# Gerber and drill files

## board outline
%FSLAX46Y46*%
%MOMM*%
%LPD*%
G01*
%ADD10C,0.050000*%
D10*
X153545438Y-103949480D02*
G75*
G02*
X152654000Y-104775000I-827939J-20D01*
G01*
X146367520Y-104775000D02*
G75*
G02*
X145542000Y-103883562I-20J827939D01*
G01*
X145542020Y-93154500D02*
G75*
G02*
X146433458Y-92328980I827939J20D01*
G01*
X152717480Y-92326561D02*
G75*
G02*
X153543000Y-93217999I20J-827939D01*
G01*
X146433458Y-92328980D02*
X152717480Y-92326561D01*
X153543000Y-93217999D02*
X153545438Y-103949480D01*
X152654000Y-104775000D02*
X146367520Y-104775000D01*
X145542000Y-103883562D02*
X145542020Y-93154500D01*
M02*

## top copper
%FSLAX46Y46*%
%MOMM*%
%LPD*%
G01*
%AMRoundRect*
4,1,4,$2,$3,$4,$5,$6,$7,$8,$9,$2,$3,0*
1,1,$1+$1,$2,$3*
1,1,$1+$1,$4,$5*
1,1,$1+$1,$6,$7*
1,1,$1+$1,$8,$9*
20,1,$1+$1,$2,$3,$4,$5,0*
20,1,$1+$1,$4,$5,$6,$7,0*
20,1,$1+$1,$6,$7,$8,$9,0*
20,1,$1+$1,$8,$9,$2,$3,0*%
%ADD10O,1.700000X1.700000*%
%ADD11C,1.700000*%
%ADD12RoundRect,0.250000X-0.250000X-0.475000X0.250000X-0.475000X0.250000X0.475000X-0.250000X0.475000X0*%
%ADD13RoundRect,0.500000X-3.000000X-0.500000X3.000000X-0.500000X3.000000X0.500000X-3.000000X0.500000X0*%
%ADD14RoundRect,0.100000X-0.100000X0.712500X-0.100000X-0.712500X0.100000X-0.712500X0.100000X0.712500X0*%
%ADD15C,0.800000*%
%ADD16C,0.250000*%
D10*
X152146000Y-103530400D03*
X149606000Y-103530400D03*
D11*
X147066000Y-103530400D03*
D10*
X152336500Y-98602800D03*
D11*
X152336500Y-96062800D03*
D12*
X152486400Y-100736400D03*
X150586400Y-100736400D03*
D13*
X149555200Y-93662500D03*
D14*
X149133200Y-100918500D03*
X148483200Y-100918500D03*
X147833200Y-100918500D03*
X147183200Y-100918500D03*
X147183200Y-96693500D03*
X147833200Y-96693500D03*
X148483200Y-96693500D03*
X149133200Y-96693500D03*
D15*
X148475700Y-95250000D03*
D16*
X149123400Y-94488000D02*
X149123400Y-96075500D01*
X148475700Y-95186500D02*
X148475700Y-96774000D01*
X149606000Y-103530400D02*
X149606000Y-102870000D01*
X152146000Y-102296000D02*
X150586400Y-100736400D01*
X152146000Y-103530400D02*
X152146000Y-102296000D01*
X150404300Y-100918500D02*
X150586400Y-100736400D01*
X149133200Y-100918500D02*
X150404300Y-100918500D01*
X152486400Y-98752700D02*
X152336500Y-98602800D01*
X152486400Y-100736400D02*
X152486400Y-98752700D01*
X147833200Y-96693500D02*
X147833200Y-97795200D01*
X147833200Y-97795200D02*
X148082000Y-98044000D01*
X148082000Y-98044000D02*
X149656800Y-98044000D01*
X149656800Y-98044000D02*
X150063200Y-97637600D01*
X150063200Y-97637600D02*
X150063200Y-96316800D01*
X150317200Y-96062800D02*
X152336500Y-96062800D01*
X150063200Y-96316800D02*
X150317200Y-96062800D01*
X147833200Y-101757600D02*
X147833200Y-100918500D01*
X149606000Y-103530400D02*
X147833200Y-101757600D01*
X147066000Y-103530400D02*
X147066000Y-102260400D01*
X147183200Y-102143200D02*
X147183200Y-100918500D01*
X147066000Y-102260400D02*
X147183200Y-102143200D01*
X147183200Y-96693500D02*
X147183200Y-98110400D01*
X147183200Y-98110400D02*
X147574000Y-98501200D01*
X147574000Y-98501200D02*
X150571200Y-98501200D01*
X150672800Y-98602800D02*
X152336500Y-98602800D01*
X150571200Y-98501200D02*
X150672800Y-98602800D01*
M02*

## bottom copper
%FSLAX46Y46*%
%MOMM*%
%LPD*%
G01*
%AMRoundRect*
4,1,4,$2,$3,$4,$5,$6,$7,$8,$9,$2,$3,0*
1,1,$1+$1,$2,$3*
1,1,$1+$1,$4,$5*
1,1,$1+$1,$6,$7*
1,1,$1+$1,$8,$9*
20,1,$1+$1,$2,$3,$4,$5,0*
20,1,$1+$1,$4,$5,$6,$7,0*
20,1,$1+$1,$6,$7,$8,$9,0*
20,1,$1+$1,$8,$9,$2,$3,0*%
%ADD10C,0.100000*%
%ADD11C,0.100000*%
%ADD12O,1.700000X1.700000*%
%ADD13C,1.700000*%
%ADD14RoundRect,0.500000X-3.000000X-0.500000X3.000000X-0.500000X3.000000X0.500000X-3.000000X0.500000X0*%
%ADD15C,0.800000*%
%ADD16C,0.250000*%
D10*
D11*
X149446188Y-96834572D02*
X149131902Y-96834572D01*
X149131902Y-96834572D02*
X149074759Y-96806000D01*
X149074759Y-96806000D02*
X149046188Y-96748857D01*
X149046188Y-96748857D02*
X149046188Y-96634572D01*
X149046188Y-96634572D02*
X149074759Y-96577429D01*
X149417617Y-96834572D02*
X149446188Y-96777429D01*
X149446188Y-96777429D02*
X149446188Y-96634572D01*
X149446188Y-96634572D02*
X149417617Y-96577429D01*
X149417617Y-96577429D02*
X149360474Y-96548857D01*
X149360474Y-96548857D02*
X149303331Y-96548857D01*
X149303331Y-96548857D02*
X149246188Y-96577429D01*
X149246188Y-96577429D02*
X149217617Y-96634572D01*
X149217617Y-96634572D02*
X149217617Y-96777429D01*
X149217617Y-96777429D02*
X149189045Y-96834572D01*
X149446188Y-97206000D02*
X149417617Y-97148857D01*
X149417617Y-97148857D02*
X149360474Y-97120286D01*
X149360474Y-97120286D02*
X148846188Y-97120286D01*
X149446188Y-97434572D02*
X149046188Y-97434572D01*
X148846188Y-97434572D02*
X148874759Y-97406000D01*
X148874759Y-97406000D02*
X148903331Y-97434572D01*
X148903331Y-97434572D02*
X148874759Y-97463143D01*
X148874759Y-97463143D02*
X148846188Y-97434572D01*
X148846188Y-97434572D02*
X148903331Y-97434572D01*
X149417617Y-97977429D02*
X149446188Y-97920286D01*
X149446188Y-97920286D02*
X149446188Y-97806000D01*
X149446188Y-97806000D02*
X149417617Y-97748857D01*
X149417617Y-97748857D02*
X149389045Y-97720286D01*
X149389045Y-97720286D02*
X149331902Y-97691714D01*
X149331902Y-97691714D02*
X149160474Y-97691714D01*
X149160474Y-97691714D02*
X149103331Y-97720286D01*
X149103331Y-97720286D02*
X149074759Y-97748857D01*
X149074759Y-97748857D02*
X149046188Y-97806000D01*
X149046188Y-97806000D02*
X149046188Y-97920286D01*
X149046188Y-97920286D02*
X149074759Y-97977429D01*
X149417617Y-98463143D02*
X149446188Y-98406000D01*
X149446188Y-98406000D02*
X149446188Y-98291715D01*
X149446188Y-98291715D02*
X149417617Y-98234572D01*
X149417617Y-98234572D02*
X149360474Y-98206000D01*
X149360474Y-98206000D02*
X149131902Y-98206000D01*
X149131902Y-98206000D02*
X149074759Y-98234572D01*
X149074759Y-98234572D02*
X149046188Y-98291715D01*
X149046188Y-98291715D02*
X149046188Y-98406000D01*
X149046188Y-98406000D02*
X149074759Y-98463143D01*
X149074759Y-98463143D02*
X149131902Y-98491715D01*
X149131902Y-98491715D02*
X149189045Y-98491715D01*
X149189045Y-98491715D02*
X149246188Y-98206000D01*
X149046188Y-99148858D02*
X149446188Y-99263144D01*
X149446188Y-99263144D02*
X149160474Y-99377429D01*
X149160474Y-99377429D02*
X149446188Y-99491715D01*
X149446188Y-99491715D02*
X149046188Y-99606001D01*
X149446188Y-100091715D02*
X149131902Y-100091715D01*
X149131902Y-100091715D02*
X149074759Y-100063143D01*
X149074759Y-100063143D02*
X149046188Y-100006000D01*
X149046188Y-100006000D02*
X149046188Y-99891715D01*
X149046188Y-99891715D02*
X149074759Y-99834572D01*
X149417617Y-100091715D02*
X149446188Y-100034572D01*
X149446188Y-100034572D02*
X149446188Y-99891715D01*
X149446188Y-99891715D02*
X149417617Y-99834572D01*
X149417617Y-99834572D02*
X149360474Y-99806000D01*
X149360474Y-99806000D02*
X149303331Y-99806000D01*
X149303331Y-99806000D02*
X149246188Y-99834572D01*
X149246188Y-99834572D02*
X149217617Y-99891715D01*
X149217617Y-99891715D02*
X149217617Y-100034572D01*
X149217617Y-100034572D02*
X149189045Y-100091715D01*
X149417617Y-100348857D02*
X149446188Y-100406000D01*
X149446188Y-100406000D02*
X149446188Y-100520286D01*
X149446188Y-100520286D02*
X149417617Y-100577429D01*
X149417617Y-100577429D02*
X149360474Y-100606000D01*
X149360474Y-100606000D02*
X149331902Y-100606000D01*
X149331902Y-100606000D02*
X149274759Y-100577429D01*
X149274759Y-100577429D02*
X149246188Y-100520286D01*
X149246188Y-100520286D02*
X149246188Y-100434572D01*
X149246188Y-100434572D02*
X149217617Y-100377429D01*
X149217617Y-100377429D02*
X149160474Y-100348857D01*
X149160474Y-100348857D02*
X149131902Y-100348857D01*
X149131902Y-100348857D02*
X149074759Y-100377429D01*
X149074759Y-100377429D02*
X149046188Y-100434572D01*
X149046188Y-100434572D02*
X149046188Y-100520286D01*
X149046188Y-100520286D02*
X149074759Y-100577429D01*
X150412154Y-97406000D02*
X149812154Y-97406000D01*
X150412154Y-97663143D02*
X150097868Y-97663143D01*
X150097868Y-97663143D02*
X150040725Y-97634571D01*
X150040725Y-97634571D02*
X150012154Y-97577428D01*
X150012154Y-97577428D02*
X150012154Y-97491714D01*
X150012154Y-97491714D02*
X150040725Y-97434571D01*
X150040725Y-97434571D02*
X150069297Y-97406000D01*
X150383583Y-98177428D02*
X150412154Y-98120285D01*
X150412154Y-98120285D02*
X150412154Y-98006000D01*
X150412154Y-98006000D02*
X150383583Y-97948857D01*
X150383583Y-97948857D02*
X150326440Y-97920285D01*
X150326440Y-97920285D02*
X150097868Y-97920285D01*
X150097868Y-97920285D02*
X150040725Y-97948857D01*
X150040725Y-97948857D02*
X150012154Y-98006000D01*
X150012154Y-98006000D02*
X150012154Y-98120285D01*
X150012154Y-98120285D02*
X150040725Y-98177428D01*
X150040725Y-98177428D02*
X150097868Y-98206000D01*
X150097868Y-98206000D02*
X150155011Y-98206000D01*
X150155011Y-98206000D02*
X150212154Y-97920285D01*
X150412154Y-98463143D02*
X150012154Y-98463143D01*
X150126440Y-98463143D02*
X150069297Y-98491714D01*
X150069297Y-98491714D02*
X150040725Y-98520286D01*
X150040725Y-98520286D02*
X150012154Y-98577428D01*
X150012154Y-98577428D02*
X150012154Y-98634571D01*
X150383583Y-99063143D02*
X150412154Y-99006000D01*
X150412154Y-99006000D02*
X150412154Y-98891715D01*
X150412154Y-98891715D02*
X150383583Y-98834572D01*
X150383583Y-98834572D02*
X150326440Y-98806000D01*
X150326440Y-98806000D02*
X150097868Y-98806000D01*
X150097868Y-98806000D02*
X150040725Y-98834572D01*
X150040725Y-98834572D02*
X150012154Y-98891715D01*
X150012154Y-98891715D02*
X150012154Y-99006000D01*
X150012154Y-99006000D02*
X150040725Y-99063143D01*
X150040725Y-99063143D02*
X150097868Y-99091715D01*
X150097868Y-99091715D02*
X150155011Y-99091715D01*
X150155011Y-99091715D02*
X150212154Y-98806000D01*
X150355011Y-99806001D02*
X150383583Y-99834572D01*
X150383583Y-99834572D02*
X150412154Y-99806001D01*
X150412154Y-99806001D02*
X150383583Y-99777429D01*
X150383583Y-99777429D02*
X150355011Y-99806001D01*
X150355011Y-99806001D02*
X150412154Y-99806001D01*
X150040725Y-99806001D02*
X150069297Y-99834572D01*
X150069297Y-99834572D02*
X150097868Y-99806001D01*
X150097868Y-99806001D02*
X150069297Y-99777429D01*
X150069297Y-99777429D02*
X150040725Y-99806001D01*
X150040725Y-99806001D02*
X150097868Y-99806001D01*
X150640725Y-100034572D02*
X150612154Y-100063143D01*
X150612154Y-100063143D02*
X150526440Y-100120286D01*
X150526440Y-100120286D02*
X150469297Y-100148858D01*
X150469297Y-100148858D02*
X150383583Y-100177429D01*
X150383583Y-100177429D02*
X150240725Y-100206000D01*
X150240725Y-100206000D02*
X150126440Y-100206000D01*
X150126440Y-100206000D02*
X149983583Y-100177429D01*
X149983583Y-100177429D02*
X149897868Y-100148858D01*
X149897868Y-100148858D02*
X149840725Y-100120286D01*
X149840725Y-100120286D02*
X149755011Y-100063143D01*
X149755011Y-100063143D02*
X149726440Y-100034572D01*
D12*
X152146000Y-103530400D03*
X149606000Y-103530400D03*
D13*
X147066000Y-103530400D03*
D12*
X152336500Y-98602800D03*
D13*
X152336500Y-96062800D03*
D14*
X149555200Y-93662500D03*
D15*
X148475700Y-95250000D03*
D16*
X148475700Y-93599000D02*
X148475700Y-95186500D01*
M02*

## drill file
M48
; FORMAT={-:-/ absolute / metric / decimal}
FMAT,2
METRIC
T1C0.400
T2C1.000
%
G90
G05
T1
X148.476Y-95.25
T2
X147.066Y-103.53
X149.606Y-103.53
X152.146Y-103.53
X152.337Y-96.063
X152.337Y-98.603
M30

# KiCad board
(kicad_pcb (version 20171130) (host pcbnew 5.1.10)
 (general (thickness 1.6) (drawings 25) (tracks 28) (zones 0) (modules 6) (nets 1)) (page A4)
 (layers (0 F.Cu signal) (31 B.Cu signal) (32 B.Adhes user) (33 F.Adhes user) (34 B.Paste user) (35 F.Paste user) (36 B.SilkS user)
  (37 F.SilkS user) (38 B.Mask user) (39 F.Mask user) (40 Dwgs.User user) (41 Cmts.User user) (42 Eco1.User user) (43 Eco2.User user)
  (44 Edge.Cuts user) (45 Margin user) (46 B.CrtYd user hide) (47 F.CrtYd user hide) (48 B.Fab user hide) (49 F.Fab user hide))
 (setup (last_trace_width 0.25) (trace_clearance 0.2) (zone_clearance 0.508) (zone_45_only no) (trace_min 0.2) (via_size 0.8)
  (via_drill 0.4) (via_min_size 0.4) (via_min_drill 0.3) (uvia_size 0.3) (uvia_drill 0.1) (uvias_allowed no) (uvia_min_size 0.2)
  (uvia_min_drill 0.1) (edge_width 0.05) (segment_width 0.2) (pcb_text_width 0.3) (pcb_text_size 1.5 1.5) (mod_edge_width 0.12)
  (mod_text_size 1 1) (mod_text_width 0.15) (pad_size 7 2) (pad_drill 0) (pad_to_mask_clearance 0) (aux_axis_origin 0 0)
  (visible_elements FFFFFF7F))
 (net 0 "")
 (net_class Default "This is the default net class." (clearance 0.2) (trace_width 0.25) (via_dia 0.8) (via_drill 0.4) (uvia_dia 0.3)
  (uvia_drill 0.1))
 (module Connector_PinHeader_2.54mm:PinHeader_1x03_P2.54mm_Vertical (layer F.Cu) (at 147.066 103.5304 90)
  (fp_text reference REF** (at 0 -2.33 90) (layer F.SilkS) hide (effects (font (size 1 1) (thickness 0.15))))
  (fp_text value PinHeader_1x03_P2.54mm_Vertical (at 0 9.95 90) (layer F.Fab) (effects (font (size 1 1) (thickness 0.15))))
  (pad 3 thru_hole oval (at 0 5.08 90) (size 1.7 1.7) (drill 1) (layers *.Cu *.Mask))
  (pad 2 thru_hole oval (at 0 2.54 90) (size 1.7 1.7) (drill 1) (layers *.Cu *.Mask))
  (pad 1 thru_hole circle (at 0 0 90) (size 1.7 1.7) (drill 1) (layers *.Cu *.Mask)))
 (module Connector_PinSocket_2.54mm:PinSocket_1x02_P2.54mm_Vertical (layer F.Cu) (at 152.3365 96.0628)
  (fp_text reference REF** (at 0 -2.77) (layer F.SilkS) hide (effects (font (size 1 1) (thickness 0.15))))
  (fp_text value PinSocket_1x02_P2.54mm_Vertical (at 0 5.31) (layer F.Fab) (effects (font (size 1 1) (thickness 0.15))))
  (pad 2 thru_hole oval (at 0 2.54) (size 1.7 1.7) (drill 1) (layers *.Cu *.Mask))
  (pad 1 thru_hole circle (at 0 0) (size 1.7 1.7) (drill 1) (layers *.Cu *.Mask)))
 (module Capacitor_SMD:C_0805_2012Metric (layer F.Cu) (at 151.5364 100.7364)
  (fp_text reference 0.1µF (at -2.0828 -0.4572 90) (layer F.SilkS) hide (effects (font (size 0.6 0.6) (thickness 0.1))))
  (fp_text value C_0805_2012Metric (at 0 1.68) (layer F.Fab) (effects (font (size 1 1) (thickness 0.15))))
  (pad 2 smd roundrect (at 0.95 0) (size 1 1.45) (layers F.Cu F.Paste F.Mask) (roundrect_rratio 0.25))
  (pad 1 smd roundrect (at -0.95 0) (size 1 1.45) (layers F.Cu F.Paste F.Mask) (roundrect_rratio 0.25)))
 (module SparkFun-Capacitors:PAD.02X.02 (layer B.Cu) (at 149.5552 93.6625)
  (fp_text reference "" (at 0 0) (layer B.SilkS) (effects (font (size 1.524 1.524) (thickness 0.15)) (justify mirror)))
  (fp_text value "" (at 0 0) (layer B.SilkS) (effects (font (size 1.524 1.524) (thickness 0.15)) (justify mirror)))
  (pad P$1 smd roundrect (at 0 0) (size 7 2) (layers B.Cu B.Paste B.Mask) (roundrect_rratio 0.25)))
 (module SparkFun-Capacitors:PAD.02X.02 (layer F.Cu) (at 149.5552 93.6625)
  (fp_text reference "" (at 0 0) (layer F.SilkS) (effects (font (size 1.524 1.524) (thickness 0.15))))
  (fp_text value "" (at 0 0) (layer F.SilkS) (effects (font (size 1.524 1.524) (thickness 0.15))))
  (pad P$1 smd roundrect (at 0 0) (size 7 2) (layers F.Cu F.Paste F.Mask) (roundrect_rratio 0.25)))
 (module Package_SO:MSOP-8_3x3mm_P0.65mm (layer F.Cu) (at 148.1582 98.806 270)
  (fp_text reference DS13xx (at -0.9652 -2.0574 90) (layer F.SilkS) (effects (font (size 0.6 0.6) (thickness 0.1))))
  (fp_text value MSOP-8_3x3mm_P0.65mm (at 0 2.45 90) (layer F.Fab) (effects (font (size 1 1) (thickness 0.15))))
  (pad 8 smd roundrect (at 2.1125 -0.975 270) (size 1.625 0.4) (layers F.Cu F.Paste F.Mask) (roundrect_rratio 0.25))
  (pad 7 smd roundrect (at 2.1125 -0.325 270) (size 1.625 0.4) (layers F.Cu F.Paste F.Mask) (roundrect_rratio 0.25))
  (pad 6 smd roundrect (at 2.1125 0.325 270) (size 1.625 0.4) (layers F.Cu F.Paste F.Mask) (roundrect_rratio 0.25))
  (pad 5 smd roundrect (at 2.1125 0.975 270) (size 1.625 0.4) (layers F.Cu F.Paste F.Mask) (roundrect_rratio 0.25))
  (pad 4 smd roundrect (at -2.1125 0.975 270) (size 1.625 0.4) (layers F.Cu F.Paste F.Mask) (roundrect_rratio 0.25))
  (pad 3 smd roundrect (at -2.1125 0.325 270) (size 1.625 0.4) (layers F.Cu F.Paste F.Mask) (roundrect_rratio 0.25))
  (pad 2 smd roundrect (at -2.1125 -0.325 270) (size 1.625 0.4) (layers F.Cu F.Paste F.Mask) (roundrect_rratio 0.25))
  (pad 1 smd roundrect (at -2.1125 -0.975 270) (size 1.625 0.4) (layers F.Cu F.Paste F.Mask) (roundrect_rratio 0.25)))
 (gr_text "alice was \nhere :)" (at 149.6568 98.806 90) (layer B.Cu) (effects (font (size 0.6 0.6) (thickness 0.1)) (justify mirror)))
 (gr_arc (start 152.717499 103.9495) (end 152.654 104.775) (angle -94.4) (layer Edge.Cuts) (width 0.05))
 (gr_arc (start 146.3675 103.947061) (end 145.542 103.883562) (angle -94.4) (layer Edge.Cuts) (width 0.05))
 (gr_arc (start 146.369959 93.15448) (end 146.433458 92.32898) (angle -94.4) (layer Edge.Cuts) (width 0.05))
 (gr_arc (start 152.7175 93.1545) (end 153.543 93.217999) (angle -94.4) (layer Edge.Cuts) (width 0.05))
 (gr_line (start 146.433458 92.32898) (end 152.71748 92.326561) (layer Edge.Cuts) (width 0.05))
 (gr_line (start 153.543 93.217999) (end 153.545438 103.94948) (layer Edge.Cuts) (width 0.05))
 (gr_line (start 152.654 104.775) (end 146.36752 104.775) (layer Edge.Cuts) (width 0.05))
 (gr_line (start 145.542 103.883562) (end 145.54202 93.1545) (layer Edge.Cuts) (width 0.05))
 (segment (start 149.1234 94.488) (end 149.1234 96.0755) (width 0.25) (layer F.Cu) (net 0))
 (segment (start 148.4757 93.599) (end 148.4757 95.1865) (width 0.25) (layer B.Cu) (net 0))
 (via (at 148.4757 95.25) (size 0.8) (drill 0.4) (layers F.Cu B.Cu) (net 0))
 (segment (start 148.4757 95.1865) (end 148.4757 96.774) (width 0.25) (layer F.Cu) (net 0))
 (segment (start 149.606 103.5304) (end 149.606 102.87) (width 0.25) (layer F.Cu) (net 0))
 (segment (start 152.146 102.296) (end 150.5864 100.7364) (width 0.25) (layer F.Cu) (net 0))
 (segment (start 152.146 103.5304) (end 152.146 102.296) (width 0.25) (layer F.Cu) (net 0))
 (segment (start 150.4043 100.9185) (end 150.5864 100.7364) (width 0.25) (layer F.Cu) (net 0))
 (segment (start 149.1332 100.9185) (end 150.4043 100.9185) (width 0.25) (layer F.Cu) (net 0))
 (segment (start 152.4864 98.7527) (end 152.3365 98.6028) (width 0.25) (layer F.Cu) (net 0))
 (segment (start 152.4864 100.7364) (end 152.4864 98.7527) (width 0.25) (layer F.Cu) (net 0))
 (segment (start 147.8332 96.6935) (end 147.8332 97.7952) (width 0.25) (layer F.Cu) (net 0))
 (segment (start 147.8332 97.7952) (end 148.082 98.044) (width 0.25) (layer F.Cu) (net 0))
 (segment (start 148.082 98.044) (end 149.6568 98.044) (width 0.25) (layer F.Cu) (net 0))
 (segment (start 149.6568 98.044) (end 150.0632 97.6376) (width 0.25) (layer F.Cu) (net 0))
 (segment (start 150.0632 97.6376) (end 150.0632 96.3168) (width 0.25) (layer F.Cu) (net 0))
 (segment (start 150.3172 96.0628) (end 152.3365 96.0628) (width 0.25) (layer F.Cu) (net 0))
 (segment (start 150.0632 96.3168) (end 150.3172 96.0628) (width 0.25) (layer F.Cu) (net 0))
 (segment (start 147.8332 101.7576) (end 147.8332 100.9185) (width 0.25) (layer F.Cu) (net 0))
 (segment (start 149.606 103.5304) (end 147.8332 101.7576) (width 0.25) (layer F.Cu) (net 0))
 (segment (start 147.066 103.5304) (end 147.066 102.2604) (width 0.25) (layer F.Cu) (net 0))
 (segment (start 147.1832 102.1432) (end 147.1832 100.9185) (width 0.25) (layer F.Cu) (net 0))
 (segment (start 147.066 102.2604) (end 147.1832 102.1432) (width 0.25) (layer F.Cu) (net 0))
 (segment (start 147.1832 96.6935) (end 147.1832 98.1104) (width 0.25) (layer F.Cu) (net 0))
 (segment (start 147.1832 98.1104) (end 147.574 98.5012) (width 0.25) (layer F.Cu) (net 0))
 (segment (start 147.574 98.5012) (end 150.5712 98.5012) (width 0.25) (layer F.Cu) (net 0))
 (segment (start 150.6728 98.6028) (end 152.3365 98.6028) (width 0.25) (layer F.Cu) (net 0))
 (segment (start 150.5712 98.5012) (end 150.6728 98.6028) (width 0.25) (layer F.Cu) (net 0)))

